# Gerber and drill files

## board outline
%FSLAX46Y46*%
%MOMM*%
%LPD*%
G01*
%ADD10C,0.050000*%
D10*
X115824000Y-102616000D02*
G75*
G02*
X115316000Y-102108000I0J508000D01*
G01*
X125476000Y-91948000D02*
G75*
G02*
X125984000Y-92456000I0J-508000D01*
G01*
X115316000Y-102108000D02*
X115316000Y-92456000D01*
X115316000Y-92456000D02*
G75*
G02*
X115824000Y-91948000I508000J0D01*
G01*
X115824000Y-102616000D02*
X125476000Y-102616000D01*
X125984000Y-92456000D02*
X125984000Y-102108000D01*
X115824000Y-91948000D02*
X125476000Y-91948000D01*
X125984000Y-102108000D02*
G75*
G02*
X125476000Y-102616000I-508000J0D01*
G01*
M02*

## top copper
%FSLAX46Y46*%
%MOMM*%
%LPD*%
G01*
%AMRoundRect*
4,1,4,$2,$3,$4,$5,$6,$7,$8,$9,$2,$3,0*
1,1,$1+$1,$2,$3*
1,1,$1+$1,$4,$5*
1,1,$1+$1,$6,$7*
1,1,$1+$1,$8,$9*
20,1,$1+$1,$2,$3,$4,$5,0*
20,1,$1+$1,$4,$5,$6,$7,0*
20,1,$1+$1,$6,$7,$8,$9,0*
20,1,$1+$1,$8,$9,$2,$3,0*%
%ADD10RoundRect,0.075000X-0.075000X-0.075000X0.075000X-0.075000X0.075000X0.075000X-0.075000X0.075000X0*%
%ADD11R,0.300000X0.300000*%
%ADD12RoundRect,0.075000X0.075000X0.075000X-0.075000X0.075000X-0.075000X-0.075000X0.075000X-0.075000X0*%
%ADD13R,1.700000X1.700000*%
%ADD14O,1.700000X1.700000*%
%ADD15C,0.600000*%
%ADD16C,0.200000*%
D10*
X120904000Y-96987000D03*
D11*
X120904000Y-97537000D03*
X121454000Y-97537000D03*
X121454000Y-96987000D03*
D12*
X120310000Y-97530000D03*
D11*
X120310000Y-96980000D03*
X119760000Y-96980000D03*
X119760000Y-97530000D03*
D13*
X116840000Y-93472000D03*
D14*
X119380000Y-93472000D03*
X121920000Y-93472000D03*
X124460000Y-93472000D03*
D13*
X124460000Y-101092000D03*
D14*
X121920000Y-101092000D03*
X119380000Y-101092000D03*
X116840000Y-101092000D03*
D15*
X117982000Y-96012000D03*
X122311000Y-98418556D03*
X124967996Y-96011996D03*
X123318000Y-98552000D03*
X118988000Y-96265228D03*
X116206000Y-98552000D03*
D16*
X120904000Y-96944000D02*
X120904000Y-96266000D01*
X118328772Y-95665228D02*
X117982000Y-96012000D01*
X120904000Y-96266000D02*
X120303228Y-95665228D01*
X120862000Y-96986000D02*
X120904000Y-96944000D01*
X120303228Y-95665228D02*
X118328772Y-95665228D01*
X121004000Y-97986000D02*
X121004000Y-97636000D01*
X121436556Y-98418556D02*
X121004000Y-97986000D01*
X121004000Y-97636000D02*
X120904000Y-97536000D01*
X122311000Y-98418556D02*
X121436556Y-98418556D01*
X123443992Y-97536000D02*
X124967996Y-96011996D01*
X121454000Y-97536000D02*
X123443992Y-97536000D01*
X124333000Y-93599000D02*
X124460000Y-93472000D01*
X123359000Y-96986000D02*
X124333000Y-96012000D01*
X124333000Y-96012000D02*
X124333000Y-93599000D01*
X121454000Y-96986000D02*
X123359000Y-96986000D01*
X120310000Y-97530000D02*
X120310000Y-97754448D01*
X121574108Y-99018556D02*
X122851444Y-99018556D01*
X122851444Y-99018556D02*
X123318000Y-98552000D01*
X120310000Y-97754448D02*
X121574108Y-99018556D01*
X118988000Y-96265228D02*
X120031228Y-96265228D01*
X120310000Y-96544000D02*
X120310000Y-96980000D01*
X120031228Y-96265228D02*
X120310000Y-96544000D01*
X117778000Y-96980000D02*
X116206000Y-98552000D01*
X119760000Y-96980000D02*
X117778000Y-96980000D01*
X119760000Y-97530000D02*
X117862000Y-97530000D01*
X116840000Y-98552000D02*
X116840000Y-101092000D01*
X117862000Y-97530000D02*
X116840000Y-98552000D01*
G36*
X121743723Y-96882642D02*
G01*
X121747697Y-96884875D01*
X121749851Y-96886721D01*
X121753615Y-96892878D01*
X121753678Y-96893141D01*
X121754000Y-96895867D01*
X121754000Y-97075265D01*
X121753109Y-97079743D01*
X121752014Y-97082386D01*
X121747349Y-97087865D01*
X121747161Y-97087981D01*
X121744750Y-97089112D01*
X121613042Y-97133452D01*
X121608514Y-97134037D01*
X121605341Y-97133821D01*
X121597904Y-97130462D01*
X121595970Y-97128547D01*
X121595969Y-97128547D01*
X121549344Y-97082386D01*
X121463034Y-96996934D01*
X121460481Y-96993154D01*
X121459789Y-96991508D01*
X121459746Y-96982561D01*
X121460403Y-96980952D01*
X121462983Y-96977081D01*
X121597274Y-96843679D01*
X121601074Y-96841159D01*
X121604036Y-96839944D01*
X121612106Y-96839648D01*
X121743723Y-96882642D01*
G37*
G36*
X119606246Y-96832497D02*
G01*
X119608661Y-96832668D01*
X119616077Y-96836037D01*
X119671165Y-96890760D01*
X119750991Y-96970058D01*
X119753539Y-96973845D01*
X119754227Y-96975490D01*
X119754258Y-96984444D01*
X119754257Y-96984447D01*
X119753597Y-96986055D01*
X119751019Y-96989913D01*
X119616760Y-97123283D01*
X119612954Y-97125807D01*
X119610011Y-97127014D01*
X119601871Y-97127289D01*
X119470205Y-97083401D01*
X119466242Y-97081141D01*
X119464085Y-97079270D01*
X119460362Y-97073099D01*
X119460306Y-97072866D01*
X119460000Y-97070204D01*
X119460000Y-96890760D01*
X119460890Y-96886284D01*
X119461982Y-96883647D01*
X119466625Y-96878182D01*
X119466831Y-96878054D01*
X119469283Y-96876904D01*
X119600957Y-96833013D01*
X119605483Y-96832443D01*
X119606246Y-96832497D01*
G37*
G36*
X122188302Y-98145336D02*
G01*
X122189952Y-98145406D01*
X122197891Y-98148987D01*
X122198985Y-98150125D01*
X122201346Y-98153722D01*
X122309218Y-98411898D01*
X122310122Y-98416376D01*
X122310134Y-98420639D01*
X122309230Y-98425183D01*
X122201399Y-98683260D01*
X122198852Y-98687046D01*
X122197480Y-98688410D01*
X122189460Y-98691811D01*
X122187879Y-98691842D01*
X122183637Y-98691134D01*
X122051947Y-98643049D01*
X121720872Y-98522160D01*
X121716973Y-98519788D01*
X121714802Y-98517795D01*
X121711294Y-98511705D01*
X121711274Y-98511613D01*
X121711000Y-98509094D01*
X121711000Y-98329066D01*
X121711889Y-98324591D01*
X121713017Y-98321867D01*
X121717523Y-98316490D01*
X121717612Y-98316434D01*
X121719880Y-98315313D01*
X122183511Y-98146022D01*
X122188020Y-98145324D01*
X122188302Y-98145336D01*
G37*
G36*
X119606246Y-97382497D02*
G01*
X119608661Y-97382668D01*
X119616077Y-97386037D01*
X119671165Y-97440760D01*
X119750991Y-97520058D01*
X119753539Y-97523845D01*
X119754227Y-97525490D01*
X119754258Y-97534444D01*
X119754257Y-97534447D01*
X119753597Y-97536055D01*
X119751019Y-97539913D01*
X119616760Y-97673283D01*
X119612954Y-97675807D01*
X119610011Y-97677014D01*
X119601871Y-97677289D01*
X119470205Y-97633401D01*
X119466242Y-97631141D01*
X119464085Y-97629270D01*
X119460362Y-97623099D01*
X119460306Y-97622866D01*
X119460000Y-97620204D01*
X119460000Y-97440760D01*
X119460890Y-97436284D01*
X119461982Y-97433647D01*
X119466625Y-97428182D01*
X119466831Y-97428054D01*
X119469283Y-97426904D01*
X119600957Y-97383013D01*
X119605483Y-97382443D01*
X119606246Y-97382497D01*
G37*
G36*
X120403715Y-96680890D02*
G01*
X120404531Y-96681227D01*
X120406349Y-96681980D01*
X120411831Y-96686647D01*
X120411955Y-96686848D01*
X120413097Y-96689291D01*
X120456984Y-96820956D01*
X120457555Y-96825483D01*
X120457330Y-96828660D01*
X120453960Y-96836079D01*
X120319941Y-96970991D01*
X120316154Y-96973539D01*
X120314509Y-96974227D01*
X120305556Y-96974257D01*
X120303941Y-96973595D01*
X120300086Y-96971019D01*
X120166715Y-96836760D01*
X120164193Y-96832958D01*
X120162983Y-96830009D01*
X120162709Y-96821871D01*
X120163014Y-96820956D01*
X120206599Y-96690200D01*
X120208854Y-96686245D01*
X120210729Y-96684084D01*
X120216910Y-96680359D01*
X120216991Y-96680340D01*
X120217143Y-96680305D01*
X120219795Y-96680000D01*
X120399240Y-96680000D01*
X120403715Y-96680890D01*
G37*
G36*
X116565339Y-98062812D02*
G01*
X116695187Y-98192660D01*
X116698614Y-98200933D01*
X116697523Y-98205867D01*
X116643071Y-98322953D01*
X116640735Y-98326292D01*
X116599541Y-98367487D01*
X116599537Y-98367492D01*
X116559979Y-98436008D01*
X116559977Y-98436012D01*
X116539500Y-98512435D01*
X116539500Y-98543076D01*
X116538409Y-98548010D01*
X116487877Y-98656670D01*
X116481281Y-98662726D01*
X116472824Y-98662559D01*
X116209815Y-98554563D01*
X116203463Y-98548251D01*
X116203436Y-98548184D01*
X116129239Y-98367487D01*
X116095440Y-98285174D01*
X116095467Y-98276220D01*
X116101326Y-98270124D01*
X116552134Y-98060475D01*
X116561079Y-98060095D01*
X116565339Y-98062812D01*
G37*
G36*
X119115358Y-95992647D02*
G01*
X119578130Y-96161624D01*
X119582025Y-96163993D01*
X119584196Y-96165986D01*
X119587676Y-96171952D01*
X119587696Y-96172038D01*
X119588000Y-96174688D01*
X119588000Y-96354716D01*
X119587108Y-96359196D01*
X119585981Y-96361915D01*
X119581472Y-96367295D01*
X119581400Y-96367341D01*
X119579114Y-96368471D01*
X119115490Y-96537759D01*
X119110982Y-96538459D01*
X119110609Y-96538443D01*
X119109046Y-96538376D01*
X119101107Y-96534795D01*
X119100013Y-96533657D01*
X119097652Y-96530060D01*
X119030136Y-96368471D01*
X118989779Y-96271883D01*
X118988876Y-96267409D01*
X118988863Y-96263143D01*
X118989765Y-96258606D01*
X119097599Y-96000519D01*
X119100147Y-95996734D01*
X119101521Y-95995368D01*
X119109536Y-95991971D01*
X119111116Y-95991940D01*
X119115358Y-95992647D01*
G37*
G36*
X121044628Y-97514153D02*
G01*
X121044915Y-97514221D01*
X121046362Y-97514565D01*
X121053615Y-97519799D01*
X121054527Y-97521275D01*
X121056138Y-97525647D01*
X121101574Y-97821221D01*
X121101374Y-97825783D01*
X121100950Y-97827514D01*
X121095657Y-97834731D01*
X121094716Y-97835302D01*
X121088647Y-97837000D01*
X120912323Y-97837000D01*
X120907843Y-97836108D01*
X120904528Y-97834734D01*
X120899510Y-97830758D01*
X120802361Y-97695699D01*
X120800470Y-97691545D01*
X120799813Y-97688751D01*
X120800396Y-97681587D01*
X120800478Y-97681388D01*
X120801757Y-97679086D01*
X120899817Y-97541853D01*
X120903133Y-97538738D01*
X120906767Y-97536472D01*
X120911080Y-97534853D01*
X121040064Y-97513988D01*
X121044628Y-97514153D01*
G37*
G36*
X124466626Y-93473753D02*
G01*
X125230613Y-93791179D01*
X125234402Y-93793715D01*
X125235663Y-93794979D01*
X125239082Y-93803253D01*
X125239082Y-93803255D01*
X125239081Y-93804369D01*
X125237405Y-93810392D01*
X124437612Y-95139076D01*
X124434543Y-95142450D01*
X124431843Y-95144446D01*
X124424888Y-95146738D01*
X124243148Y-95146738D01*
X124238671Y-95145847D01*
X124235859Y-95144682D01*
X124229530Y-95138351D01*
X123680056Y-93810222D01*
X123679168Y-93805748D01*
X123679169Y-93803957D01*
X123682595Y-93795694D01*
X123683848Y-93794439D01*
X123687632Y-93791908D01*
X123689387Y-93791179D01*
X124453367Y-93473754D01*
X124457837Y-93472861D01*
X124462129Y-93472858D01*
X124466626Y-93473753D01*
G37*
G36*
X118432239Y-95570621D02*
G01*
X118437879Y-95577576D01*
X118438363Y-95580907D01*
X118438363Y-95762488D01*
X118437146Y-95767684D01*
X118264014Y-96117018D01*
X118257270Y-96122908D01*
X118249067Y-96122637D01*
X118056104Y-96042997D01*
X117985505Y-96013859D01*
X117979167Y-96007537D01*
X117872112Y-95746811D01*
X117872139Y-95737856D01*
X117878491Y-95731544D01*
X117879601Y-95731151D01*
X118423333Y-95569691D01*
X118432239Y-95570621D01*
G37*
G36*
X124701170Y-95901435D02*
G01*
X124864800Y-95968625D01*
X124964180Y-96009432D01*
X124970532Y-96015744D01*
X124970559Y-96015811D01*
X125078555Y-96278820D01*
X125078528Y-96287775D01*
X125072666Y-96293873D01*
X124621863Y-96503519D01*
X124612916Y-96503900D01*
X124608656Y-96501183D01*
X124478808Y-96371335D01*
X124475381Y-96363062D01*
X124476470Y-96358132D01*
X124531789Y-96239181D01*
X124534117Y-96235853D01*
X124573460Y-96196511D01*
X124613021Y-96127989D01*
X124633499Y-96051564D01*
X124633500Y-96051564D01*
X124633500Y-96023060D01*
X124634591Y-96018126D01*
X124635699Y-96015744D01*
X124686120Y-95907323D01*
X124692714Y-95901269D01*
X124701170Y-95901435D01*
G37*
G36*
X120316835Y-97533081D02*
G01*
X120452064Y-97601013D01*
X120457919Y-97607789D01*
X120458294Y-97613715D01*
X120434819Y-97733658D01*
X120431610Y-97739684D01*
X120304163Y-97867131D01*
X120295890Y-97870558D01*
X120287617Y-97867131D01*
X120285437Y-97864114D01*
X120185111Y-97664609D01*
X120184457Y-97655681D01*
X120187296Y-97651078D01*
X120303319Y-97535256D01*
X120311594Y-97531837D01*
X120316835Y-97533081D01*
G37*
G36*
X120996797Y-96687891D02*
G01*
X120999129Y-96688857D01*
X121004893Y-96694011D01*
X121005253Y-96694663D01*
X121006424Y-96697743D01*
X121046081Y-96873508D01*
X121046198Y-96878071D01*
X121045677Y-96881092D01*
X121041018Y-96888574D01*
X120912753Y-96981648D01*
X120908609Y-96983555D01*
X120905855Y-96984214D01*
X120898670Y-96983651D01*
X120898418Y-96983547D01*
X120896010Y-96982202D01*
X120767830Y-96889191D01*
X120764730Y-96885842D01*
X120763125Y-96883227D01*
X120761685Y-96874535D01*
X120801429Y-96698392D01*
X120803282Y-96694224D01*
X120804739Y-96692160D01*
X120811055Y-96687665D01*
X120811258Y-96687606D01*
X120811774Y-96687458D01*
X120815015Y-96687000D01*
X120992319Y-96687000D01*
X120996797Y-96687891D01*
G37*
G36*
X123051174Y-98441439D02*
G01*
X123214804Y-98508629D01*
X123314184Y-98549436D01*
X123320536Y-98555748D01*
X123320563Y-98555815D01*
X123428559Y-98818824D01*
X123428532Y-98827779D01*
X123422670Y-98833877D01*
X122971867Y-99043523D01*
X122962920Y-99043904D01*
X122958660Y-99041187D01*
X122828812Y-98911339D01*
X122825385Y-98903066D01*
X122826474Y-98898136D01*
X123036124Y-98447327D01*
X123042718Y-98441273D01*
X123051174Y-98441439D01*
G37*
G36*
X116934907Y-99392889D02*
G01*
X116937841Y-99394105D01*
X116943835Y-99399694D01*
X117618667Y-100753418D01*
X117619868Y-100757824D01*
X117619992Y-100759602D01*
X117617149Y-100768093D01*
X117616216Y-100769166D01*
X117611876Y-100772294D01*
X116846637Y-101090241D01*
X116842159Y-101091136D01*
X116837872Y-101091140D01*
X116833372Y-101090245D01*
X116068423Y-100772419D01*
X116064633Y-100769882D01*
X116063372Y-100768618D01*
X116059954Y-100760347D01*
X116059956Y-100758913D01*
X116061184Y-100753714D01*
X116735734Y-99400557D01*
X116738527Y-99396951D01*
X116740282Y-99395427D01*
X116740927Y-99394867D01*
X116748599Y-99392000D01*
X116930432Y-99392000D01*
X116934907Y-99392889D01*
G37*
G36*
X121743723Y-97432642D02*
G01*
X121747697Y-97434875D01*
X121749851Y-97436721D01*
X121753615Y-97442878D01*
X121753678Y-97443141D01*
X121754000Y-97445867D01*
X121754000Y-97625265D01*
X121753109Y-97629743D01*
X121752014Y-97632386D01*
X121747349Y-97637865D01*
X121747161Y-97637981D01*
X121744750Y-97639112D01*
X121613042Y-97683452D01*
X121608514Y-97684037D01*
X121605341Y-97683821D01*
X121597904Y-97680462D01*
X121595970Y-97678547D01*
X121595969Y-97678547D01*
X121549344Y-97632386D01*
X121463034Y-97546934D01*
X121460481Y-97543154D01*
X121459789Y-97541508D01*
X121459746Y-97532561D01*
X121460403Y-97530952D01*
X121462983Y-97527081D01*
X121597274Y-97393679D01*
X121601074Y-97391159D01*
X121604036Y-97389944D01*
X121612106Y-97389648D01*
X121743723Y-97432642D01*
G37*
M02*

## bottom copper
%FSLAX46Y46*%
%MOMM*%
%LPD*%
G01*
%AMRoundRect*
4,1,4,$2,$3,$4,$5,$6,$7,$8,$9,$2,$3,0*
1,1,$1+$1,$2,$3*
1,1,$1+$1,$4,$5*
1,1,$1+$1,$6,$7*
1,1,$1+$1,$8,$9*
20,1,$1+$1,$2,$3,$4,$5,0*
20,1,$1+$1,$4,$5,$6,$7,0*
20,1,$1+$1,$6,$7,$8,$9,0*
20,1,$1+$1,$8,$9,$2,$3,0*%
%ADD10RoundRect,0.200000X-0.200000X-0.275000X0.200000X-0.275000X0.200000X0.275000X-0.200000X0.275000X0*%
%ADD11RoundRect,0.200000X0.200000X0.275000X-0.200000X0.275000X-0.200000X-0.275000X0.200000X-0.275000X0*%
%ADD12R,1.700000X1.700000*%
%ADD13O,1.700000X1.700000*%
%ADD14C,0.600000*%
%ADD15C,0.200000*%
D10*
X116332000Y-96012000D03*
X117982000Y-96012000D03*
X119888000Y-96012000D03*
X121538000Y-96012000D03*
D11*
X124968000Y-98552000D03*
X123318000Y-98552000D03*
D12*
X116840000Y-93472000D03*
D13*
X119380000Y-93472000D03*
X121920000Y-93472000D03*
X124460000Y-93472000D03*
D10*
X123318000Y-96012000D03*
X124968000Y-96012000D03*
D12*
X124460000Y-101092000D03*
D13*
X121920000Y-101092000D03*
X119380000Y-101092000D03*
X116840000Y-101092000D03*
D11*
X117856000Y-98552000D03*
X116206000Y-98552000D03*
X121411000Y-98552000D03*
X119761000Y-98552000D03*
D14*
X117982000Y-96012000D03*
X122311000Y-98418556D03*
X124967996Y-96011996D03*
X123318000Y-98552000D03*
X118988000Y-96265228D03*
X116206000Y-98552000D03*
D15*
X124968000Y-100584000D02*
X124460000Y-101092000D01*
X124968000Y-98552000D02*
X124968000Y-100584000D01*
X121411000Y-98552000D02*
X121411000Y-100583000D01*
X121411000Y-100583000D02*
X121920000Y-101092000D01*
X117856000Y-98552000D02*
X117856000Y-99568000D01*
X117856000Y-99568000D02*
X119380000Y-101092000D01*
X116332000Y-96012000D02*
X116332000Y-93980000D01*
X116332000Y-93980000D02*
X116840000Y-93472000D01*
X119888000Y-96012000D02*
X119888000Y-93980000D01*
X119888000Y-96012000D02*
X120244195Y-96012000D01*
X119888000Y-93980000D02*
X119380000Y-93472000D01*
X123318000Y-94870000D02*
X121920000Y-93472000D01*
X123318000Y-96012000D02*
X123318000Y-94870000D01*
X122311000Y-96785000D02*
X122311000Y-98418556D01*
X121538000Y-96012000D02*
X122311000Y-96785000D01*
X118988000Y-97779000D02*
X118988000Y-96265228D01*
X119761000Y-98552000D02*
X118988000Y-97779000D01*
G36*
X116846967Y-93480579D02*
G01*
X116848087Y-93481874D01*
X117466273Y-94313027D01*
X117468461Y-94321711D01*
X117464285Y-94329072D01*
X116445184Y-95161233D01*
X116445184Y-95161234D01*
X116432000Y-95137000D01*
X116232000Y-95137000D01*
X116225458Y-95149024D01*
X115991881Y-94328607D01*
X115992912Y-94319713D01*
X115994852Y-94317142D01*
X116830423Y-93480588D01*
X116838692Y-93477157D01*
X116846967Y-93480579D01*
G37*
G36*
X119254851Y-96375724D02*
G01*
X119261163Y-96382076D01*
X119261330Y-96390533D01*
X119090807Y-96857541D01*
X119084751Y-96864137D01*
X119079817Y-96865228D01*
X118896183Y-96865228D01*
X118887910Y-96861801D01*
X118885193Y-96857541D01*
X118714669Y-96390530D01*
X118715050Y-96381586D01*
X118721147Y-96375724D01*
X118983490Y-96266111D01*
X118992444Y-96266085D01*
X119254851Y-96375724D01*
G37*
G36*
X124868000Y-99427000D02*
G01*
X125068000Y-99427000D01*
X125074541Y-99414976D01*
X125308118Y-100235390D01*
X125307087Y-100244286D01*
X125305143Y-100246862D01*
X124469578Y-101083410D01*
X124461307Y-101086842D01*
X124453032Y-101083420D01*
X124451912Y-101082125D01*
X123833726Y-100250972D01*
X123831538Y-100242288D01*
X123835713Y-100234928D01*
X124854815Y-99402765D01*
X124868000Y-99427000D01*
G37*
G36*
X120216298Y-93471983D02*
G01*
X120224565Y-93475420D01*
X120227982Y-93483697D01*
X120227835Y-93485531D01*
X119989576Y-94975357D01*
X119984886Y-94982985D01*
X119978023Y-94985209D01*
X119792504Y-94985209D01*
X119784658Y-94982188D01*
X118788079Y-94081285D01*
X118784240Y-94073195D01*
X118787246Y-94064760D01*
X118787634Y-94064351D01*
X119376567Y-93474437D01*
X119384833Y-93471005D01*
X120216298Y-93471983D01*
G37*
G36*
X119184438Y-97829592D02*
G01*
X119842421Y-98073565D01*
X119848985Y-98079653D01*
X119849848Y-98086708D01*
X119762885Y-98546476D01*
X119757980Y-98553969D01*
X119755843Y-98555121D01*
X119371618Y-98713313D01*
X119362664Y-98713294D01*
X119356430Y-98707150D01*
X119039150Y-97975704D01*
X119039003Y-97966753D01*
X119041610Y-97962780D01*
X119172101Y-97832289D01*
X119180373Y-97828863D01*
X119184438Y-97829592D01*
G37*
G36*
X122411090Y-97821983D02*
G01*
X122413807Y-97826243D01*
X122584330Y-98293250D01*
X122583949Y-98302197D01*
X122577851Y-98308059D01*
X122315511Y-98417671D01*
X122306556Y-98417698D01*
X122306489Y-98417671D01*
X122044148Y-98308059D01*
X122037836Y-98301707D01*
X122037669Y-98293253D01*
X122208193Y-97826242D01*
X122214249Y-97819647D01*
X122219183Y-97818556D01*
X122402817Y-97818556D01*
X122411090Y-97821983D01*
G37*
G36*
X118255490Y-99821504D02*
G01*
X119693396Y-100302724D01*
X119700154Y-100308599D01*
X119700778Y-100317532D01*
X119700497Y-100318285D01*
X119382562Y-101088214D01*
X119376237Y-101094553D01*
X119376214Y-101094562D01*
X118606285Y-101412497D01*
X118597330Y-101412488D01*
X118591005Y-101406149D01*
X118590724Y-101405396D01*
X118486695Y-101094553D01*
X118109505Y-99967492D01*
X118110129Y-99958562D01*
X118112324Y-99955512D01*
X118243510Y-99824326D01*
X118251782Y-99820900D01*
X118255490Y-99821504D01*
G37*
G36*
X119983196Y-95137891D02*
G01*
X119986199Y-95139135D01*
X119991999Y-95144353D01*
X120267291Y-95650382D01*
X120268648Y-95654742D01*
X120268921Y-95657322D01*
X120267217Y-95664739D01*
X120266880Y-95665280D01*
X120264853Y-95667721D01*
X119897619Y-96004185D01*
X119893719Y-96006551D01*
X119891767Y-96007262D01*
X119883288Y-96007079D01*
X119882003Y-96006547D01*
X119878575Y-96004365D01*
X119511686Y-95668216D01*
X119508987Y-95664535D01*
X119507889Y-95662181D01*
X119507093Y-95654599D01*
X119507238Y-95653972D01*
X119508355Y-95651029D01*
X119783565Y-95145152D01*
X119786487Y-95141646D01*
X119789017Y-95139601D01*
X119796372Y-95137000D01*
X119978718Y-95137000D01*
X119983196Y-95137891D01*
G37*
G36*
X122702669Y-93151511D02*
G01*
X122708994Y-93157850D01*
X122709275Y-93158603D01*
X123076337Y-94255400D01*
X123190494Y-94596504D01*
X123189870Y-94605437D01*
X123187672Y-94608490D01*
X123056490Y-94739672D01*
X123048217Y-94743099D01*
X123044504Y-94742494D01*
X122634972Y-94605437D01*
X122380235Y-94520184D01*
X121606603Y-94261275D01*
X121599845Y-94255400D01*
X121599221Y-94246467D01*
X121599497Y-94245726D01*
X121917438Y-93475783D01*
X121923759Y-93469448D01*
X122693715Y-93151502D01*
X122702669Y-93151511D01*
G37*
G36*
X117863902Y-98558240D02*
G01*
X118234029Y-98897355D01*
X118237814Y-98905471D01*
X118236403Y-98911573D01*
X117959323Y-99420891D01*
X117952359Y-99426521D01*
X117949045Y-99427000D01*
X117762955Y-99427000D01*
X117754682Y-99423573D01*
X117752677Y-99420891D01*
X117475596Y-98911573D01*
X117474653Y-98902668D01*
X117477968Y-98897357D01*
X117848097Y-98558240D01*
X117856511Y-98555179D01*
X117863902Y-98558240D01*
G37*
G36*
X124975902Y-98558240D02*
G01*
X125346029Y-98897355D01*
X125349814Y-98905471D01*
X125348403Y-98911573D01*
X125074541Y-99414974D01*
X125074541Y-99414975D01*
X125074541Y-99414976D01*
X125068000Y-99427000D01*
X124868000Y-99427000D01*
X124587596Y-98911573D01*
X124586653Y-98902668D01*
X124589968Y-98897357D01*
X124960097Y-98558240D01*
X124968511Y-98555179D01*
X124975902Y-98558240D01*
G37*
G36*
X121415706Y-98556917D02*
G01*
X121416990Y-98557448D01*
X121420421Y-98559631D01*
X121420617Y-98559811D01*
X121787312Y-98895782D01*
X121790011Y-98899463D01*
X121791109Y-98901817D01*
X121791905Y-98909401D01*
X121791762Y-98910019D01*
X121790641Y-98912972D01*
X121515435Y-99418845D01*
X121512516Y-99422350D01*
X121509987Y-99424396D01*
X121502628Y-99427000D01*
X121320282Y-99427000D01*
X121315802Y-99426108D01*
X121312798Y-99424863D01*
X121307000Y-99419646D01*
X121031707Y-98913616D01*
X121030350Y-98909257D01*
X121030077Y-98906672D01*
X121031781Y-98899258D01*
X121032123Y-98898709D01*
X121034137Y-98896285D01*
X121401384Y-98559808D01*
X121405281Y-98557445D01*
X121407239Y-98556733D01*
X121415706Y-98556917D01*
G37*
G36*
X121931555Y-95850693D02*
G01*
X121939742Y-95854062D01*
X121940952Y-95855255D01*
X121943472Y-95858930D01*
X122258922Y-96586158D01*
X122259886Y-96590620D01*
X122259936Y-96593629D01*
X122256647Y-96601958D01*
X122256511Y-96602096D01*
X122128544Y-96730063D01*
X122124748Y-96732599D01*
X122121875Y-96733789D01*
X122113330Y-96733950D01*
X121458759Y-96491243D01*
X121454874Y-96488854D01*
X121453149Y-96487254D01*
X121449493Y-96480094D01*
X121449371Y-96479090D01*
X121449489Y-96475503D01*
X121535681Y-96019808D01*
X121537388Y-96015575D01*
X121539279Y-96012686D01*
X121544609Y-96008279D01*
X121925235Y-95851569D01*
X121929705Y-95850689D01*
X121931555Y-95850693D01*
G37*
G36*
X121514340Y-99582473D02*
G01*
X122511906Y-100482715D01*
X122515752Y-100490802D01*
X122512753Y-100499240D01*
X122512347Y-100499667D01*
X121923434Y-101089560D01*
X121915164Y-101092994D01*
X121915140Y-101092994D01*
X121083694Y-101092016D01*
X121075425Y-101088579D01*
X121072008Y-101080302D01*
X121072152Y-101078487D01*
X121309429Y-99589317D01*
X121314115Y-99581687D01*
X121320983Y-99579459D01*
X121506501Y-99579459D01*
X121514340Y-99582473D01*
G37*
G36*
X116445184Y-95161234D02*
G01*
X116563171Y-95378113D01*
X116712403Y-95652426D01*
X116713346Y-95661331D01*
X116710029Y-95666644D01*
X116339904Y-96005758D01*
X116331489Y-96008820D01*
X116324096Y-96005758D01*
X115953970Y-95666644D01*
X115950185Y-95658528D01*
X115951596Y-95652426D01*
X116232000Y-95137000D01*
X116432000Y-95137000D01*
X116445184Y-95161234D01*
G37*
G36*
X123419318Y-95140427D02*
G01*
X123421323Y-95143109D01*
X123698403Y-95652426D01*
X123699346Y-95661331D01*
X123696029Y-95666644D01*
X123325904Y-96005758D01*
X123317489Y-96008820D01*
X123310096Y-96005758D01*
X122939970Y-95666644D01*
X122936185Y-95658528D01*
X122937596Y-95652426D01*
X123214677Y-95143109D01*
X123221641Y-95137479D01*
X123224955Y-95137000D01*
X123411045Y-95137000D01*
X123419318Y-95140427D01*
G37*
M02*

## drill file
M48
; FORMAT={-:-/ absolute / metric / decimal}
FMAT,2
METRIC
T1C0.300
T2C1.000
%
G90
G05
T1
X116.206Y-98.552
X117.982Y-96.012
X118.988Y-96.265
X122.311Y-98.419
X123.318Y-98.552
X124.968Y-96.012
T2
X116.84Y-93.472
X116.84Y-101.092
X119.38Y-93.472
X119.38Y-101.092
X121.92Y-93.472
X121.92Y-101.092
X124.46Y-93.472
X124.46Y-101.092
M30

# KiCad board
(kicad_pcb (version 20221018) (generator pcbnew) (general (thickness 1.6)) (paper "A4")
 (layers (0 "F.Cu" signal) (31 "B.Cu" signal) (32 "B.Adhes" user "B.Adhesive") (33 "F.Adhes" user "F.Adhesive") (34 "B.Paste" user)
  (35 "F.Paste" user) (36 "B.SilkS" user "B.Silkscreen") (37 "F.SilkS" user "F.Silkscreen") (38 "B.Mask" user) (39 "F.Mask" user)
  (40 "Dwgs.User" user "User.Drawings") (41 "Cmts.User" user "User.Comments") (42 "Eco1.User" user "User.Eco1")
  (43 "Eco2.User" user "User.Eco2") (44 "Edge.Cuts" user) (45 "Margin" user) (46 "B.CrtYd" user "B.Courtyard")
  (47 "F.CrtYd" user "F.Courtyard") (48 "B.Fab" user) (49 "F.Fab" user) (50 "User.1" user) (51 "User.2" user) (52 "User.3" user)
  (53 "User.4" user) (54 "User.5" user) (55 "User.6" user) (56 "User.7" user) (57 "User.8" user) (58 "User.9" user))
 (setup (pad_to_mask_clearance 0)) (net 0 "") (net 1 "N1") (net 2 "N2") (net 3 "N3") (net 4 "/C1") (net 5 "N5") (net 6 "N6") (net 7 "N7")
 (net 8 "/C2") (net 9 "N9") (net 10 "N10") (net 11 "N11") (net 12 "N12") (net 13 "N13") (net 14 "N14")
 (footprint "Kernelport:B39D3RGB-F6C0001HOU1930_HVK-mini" (layer "F.Cu") (at 121.179 97.262)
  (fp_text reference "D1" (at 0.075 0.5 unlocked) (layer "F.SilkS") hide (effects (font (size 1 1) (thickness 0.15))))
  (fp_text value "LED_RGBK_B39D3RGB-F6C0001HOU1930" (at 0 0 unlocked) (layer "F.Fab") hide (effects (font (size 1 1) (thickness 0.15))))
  (pad "1" smd roundrect (at -0.275 -0.275) (size 0.3 0.3) (layers "F.Cu" "F.Paste" "F.Mask") (roundrect_rratio 0.25) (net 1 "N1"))
  (pad "2" smd rect (at -0.275 0.275) (size 0.3 0.3) (layers "F.Cu" "F.Paste" "F.Mask") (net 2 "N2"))
  (pad "3" smd rect (at 0.275 0.275) (size 0.3 0.3) (layers "F.Cu" "F.Paste" "F.Mask") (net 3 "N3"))
  (pad "4" smd rect (at 0.275 -0.275) (size 0.3 0.3) (layers "F.Cu" "F.Paste" "F.Mask") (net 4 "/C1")))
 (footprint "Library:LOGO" (layer "F.Cu") (at 123.952 97.282)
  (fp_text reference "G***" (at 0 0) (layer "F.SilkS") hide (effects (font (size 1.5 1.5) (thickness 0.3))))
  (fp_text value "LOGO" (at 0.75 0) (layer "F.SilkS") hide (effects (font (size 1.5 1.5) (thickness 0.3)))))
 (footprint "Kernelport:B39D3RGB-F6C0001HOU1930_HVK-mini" (layer "F.Cu") (at 120.035 97.255 180)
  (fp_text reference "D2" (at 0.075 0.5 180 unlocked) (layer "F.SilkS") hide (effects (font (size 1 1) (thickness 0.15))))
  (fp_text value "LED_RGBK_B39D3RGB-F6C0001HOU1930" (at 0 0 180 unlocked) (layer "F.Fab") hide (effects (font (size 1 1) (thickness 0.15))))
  (pad "1" smd roundrect (at -0.275 -0.275 180) (size 0.3 0.3) (layers "F.Cu" "F.Paste" "F.Mask") (roundrect_rratio 0.25) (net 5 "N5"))
  (pad "2" smd rect (at -0.275 0.275 180) (size 0.3 0.3) (layers "F.Cu" "F.Paste" "F.Mask") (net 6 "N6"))
  (pad "3" smd rect (at 0.275 0.275 180) (size 0.3 0.3) (layers "F.Cu" "F.Paste" "F.Mask") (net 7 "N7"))
  (pad "4" smd rect (at 0.275 -0.275 180) (size 0.3 0.3) (layers "F.Cu" "F.Paste" "F.Mask") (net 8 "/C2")))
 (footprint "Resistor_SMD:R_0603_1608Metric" (layer "B.Cu") (at 117.157 96.012)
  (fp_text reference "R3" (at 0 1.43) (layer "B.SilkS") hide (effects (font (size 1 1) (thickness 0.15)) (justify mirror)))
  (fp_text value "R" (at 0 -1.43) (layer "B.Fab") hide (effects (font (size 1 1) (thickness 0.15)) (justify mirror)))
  (pad "1" smd roundrect (at -0.825 0) (size 0.8 0.95) (layers "B.Cu" "B.Paste" "B.Mask") (roundrect_rratio 0.25) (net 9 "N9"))
  (pad "2" smd roundrect (at 0.825 0) (size 0.8 0.95) (layers "B.Cu" "B.Paste" "B.Mask") (roundrect_rratio 0.25) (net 1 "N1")))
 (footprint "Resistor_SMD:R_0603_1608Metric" (layer "B.Cu") (at 120.713 96.012)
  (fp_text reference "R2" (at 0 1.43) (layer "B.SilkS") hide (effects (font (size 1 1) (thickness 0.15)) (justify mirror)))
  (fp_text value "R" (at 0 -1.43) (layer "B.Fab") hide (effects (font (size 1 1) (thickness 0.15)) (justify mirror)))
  (pad "1" smd roundrect (at -0.825 0) (size 0.8 0.95) (layers "B.Cu" "B.Paste" "B.Mask") (roundrect_rratio 0.25) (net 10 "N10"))
  (pad "2" smd roundrect (at 0.825 0) (size 0.8 0.95) (layers "B.Cu" "B.Paste" "B.Mask") (roundrect_rratio 0.25) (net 2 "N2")))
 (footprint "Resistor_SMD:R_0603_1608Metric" (layer "B.Cu") (at 124.143 98.552 180)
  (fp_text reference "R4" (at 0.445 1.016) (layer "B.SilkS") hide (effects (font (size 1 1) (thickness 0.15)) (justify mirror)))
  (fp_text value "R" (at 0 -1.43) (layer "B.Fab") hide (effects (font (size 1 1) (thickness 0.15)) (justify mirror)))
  (pad "1" smd roundrect (at -0.825 0 180) (size 0.8 0.95) (layers "B.Cu" "B.Paste" "B.Mask") (roundrect_rratio 0.25) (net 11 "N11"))
  (pad "2" smd roundrect (at 0.825 0 180) (size 0.8 0.95) (layers "B.Cu" "B.Paste" "B.Mask") (roundrect_rratio 0.25) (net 5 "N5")))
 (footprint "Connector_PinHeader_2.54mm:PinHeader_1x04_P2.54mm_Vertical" (layer "B.Cu") (at 116.84 93.472 -90)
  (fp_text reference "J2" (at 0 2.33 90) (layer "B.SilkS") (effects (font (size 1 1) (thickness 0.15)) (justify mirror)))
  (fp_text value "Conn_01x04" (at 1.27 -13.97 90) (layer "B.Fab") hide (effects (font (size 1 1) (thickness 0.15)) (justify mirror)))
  (pad "1" thru_hole rect (at 0 0 270) (size 1.7 1.7) (drill 1) (layers "*.Cu" "*.Mask") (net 9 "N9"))
  (pad "2" thru_hole oval (at 0 -2.54 270) (size 1.7 1.7) (drill 1) (layers "*.Cu" "*.Mask") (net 10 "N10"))
  (pad "3" thru_hole oval (at 0 -5.08 270) (size 1.7 1.7) (drill 1) (layers "*.Cu" "*.Mask") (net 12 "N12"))
  (pad "4" thru_hole oval (at 0 -7.62 270) (size 1.7 1.7) (drill 1) (layers "*.Cu" "*.Mask") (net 4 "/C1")))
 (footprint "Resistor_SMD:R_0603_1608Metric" (layer "B.Cu") (at 124.143 96.012)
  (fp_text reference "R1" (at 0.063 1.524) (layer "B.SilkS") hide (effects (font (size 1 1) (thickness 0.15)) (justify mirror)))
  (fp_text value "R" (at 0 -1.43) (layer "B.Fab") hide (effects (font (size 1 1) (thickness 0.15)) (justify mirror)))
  (pad "1" smd roundrect (at -0.825 0) (size 0.8 0.95) (layers "B.Cu" "B.Paste" "B.Mask") (roundrect_rratio 0.25) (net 12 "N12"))
  (pad "2" smd roundrect (at 0.825 0) (size 0.8 0.95) (layers "B.Cu" "B.Paste" "B.Mask") (roundrect_rratio 0.25) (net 3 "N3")))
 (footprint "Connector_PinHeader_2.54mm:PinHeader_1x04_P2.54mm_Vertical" (layer "B.Cu") (at 124.46 101.092 90)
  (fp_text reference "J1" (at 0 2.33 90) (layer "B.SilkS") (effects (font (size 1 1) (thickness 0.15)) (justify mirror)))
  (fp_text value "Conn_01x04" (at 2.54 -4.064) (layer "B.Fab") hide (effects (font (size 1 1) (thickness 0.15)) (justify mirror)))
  (pad "1" thru_hole rect (at 0 0 90) (size 1.7 1.7) (drill 1) (layers "*.Cu" "*.Mask") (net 11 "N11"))
  (pad "2" thru_hole oval (at 0 -2.54 90) (size 1.7 1.7) (drill 1) (layers "*.Cu" "*.Mask") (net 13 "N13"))
  (pad "3" thru_hole oval (at 0 -5.08 90) (size 1.7 1.7) (drill 1) (layers "*.Cu" "*.Mask") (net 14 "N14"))
  (pad "4" thru_hole oval (at 0 -7.62 90) (size 1.7 1.7) (drill 1) (layers "*.Cu" "*.Mask") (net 8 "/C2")))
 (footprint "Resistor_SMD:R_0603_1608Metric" (layer "B.Cu") (at 117.031 98.552 180)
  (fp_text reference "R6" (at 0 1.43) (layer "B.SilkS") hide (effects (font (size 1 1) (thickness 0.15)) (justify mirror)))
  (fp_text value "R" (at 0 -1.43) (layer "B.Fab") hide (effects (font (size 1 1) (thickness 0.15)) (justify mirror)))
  (pad "1" smd roundrect (at -0.825 0 180) (size 0.8 0.95) (layers "B.Cu" "B.Paste" "B.Mask") (roundrect_rratio 0.25) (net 14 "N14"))
  (pad "2" smd roundrect (at 0.825 0 180) (size 0.8 0.95) (layers "B.Cu" "B.Paste" "B.Mask") (roundrect_rratio 0.25) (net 7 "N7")))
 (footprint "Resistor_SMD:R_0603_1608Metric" (layer "B.Cu") (at 120.586 98.552 180)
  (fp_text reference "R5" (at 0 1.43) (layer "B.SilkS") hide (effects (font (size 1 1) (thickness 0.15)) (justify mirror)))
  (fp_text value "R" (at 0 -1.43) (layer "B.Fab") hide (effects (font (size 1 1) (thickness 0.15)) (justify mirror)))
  (pad "1" smd roundrect (at -0.825 0 180) (size 0.8 0.95) (layers "B.Cu" "B.Paste" "B.Mask") (roundrect_rratio 0.25) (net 13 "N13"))
  (pad "2" smd roundrect (at 0.825 0 180) (size 0.8 0.95) (layers "B.Cu" "B.Paste" "B.Mask") (roundrect_rratio 0.25) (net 6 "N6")))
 (gr_arc (start 115.824 102.616) (mid 115.46479 102.46721) (end 115.316 102.108) (stroke (width 0.05) (type default)) (layer "Edge.Cuts"))
 (gr_arc (start 125.476 91.948) (mid 125.83521 92.09679) (end 125.984 92.456) (stroke (width 0.05) (type default)) (layer "Edge.Cuts"))
 (gr_line (start 115.316 102.108) (end 115.316 92.456) (stroke (width 0.05) (type default)) (layer "Edge.Cuts"))
 (gr_arc (start 115.316 92.456) (mid 115.46479 92.09679) (end 115.824 91.948) (stroke (width 0.05) (type default)) (layer "Edge.Cuts"))
 (gr_line (start 115.824 102.616) (end 125.476 102.616) (stroke (width 0.05) (type default)) (layer "Edge.Cuts"))
 (gr_line (start 125.984 92.456) (end 125.984 102.108) (stroke (width 0.05) (type default)) (layer "Edge.Cuts"))
 (gr_line (start 115.824 91.948) (end 125.476 91.948) (stroke (width 0.05) (type default)) (layer "Edge.Cuts"))
 (gr_arc (start 125.984 102.108) (mid 125.83521 102.46721) (end 125.476 102.616) (stroke (width 0.05) (type default)) (layer "Edge.Cuts"))
 (segment (start 124.968 100.584) (end 124.46 101.092) (width 0.2) (layer "B.Cu") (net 11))
 (segment (start 124.968 98.552) (end 124.968 100.584) (width 0.2) (layer "B.Cu") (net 11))
 (segment (start 121.411 98.552) (end 121.411 100.583) (width 0.2) (layer "B.Cu") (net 13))
 (segment (start 121.411 100.583) (end 121.92 101.092) (width 0.2) (layer "B.Cu") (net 13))
 (segment (start 117.856 98.552) (end 117.856 99.568) (width 0.2) (layer "B.Cu") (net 14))
 (segment (start 117.856 99.568) (end 119.38 101.092) (width 0.2) (layer "B.Cu") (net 14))
 (segment (start 116.332 96.012) (end 116.332 93.98) (width 0.2) (layer "B.Cu") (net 9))
 (segment (start 116.332 93.98) (end 116.84 93.472) (width 0.2) (layer "B.Cu") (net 9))
 (segment (start 119.888 96.012) (end 119.888 93.98) (width 0.2) (layer "B.Cu") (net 10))
 (segment (start 119.888 96.012) (end 120.244195 96.012) (width 0.2) (layer "B.Cu") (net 10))
 (segment (start 119.888 93.98) (end 119.38 93.472) (width 0.2) (layer "B.Cu") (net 10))
 (segment (start 123.318 94.87) (end 121.92 93.472) (width 0.2) (layer "B.Cu") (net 12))
 (segment (start 123.318 96.012) (end 123.318 94.87) (width 0.2) (layer "B.Cu") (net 12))
 (segment (start 120.904 96.944) (end 120.904 96.266) (width 0.2) (layer "F.Cu") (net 1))
 (segment (start 118.328772 95.665228) (end 117.982 96.012) (width 0.2) (layer "F.Cu") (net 1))
 (segment (start 120.904 96.266) (end 120.303228 95.665228) (width 0.2) (layer "F.Cu") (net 1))
 (segment (start 120.862 96.986) (end 120.904 96.944) (width 0.2) (layer "F.Cu") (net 1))
 (segment (start 120.303228 95.665228) (end 118.328772 95.665228) (width 0.2) (layer "F.Cu") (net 1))
 (via (at 117.982 96.012) (size 0.6) (drill 0.3) (layers "F.Cu" "B.Cu") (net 1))
 (segment (start 121.004 97.986) (end 121.004 97.636) (width 0.2) (layer "F.Cu") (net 2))
 (segment (start 121.436556 98.418556) (end 121.004 97.986) (width 0.2) (layer "F.Cu") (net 2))
 (segment (start 121.004 97.636) (end 120.904 97.536) (width 0.2) (layer "F.Cu") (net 2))
 (segment (start 122.311 98.418556) (end 121.436556 98.418556) (width 0.2) (layer "F.Cu") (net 2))
 (via (at 122.311 98.418556) (size 0.6) (drill 0.3) (layers "F.Cu" "B.Cu") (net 2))
 (segment (start 122.311 96.785) (end 122.311 98.418556) (width 0.2) (layer "B.Cu") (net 2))
 (segment (start 121.538 96.012) (end 122.311 96.785) (width 0.2) (layer "B.Cu") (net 2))
 (segment (start 123.443992 97.536) (end 124.967996 96.011996) (width 0.2) (layer "F.Cu") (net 3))
 (segment (start 121.454 97.536) (end 123.443992 97.536) (width 0.2) (layer "F.Cu") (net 3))
 (via (at 124.967996 96.011996) (size 0.6) (drill 0.3) (layers "F.Cu" "B.Cu") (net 3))
 (segment (start 124.333 93.599) (end 124.46 93.472) (width 0.2) (layer "F.Cu") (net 4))
 (segment (start 123.359 96.986) (end 124.333 96.012) (width 0.2) (layer "F.Cu") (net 4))
 (segment (start 124.333 96.012) (end 124.333 93.599) (width 0.2) (layer "F.Cu") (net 4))
 (segment (start 121.454 96.986) (end 123.359 96.986) (width 0.2) (layer "F.Cu") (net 4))
 (segment (start 120.31 97.53) (end 120.31 97.754448) (width 0.2) (layer "F.Cu") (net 5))
 (segment (start 121.574108 99.018556) (end 122.851444 99.018556) (width 0.2) (layer "F.Cu") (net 5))
 (segment (start 122.851444 99.018556) (end 123.318 98.552) (width 0.2) (layer "F.Cu") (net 5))
 (segment (start 120.31 97.754448) (end 121.574108 99.018556) (width 0.2) (layer "F.Cu") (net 5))
 (via (at 123.318 98.552) (size 0.6) (drill 0.3) (layers "F.Cu" "B.Cu") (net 5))
 (segment (start 118.988 96.265228) (end 120.031228 96.265228) (width 0.2) (layer "F.Cu") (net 6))
 (segment (start 120.31 96.544) (end 120.31 96.98) (width 0.2) (layer "F.Cu") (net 6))
 (segment (start 120.031228 96.265228) (end 120.31 96.544) (width 0.2) (layer "F.Cu") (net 6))
 (via (at 118.988 96.265228) (size 0.6) (drill 0.3) (layers "F.Cu" "B.Cu") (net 6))
 (segment (start 118.988 97.779) (end 118.988 96.265228) (width 0.2) (layer "B.Cu") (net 6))
 (segment (start 119.761 98.552) (end 118.988 97.779) (width 0.2) (layer "B.Cu") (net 6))
 (segment (start 117.778 96.98) (end 116.206 98.552) (width 0.2) (layer "F.Cu") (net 7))
 (segment (start 119.76 96.98) (end 117.778 96.98) (width 0.2) (layer "F.Cu") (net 7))
 (via (at 116.206 98.552) (size 0.6) (drill 0.3) (layers "F.Cu" "B.Cu") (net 7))
 (segment (start 119.76 97.53) (end 117.862 97.53) (width 0.2) (layer "F.Cu") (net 8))
 (segment (start 116.84 98.552) (end 116.84 101.092) (width 0.2) (layer "F.Cu") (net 8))
 (segment (start 117.862 97.53) (end 116.84 98.552) (width 0.2) (layer "F.Cu") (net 8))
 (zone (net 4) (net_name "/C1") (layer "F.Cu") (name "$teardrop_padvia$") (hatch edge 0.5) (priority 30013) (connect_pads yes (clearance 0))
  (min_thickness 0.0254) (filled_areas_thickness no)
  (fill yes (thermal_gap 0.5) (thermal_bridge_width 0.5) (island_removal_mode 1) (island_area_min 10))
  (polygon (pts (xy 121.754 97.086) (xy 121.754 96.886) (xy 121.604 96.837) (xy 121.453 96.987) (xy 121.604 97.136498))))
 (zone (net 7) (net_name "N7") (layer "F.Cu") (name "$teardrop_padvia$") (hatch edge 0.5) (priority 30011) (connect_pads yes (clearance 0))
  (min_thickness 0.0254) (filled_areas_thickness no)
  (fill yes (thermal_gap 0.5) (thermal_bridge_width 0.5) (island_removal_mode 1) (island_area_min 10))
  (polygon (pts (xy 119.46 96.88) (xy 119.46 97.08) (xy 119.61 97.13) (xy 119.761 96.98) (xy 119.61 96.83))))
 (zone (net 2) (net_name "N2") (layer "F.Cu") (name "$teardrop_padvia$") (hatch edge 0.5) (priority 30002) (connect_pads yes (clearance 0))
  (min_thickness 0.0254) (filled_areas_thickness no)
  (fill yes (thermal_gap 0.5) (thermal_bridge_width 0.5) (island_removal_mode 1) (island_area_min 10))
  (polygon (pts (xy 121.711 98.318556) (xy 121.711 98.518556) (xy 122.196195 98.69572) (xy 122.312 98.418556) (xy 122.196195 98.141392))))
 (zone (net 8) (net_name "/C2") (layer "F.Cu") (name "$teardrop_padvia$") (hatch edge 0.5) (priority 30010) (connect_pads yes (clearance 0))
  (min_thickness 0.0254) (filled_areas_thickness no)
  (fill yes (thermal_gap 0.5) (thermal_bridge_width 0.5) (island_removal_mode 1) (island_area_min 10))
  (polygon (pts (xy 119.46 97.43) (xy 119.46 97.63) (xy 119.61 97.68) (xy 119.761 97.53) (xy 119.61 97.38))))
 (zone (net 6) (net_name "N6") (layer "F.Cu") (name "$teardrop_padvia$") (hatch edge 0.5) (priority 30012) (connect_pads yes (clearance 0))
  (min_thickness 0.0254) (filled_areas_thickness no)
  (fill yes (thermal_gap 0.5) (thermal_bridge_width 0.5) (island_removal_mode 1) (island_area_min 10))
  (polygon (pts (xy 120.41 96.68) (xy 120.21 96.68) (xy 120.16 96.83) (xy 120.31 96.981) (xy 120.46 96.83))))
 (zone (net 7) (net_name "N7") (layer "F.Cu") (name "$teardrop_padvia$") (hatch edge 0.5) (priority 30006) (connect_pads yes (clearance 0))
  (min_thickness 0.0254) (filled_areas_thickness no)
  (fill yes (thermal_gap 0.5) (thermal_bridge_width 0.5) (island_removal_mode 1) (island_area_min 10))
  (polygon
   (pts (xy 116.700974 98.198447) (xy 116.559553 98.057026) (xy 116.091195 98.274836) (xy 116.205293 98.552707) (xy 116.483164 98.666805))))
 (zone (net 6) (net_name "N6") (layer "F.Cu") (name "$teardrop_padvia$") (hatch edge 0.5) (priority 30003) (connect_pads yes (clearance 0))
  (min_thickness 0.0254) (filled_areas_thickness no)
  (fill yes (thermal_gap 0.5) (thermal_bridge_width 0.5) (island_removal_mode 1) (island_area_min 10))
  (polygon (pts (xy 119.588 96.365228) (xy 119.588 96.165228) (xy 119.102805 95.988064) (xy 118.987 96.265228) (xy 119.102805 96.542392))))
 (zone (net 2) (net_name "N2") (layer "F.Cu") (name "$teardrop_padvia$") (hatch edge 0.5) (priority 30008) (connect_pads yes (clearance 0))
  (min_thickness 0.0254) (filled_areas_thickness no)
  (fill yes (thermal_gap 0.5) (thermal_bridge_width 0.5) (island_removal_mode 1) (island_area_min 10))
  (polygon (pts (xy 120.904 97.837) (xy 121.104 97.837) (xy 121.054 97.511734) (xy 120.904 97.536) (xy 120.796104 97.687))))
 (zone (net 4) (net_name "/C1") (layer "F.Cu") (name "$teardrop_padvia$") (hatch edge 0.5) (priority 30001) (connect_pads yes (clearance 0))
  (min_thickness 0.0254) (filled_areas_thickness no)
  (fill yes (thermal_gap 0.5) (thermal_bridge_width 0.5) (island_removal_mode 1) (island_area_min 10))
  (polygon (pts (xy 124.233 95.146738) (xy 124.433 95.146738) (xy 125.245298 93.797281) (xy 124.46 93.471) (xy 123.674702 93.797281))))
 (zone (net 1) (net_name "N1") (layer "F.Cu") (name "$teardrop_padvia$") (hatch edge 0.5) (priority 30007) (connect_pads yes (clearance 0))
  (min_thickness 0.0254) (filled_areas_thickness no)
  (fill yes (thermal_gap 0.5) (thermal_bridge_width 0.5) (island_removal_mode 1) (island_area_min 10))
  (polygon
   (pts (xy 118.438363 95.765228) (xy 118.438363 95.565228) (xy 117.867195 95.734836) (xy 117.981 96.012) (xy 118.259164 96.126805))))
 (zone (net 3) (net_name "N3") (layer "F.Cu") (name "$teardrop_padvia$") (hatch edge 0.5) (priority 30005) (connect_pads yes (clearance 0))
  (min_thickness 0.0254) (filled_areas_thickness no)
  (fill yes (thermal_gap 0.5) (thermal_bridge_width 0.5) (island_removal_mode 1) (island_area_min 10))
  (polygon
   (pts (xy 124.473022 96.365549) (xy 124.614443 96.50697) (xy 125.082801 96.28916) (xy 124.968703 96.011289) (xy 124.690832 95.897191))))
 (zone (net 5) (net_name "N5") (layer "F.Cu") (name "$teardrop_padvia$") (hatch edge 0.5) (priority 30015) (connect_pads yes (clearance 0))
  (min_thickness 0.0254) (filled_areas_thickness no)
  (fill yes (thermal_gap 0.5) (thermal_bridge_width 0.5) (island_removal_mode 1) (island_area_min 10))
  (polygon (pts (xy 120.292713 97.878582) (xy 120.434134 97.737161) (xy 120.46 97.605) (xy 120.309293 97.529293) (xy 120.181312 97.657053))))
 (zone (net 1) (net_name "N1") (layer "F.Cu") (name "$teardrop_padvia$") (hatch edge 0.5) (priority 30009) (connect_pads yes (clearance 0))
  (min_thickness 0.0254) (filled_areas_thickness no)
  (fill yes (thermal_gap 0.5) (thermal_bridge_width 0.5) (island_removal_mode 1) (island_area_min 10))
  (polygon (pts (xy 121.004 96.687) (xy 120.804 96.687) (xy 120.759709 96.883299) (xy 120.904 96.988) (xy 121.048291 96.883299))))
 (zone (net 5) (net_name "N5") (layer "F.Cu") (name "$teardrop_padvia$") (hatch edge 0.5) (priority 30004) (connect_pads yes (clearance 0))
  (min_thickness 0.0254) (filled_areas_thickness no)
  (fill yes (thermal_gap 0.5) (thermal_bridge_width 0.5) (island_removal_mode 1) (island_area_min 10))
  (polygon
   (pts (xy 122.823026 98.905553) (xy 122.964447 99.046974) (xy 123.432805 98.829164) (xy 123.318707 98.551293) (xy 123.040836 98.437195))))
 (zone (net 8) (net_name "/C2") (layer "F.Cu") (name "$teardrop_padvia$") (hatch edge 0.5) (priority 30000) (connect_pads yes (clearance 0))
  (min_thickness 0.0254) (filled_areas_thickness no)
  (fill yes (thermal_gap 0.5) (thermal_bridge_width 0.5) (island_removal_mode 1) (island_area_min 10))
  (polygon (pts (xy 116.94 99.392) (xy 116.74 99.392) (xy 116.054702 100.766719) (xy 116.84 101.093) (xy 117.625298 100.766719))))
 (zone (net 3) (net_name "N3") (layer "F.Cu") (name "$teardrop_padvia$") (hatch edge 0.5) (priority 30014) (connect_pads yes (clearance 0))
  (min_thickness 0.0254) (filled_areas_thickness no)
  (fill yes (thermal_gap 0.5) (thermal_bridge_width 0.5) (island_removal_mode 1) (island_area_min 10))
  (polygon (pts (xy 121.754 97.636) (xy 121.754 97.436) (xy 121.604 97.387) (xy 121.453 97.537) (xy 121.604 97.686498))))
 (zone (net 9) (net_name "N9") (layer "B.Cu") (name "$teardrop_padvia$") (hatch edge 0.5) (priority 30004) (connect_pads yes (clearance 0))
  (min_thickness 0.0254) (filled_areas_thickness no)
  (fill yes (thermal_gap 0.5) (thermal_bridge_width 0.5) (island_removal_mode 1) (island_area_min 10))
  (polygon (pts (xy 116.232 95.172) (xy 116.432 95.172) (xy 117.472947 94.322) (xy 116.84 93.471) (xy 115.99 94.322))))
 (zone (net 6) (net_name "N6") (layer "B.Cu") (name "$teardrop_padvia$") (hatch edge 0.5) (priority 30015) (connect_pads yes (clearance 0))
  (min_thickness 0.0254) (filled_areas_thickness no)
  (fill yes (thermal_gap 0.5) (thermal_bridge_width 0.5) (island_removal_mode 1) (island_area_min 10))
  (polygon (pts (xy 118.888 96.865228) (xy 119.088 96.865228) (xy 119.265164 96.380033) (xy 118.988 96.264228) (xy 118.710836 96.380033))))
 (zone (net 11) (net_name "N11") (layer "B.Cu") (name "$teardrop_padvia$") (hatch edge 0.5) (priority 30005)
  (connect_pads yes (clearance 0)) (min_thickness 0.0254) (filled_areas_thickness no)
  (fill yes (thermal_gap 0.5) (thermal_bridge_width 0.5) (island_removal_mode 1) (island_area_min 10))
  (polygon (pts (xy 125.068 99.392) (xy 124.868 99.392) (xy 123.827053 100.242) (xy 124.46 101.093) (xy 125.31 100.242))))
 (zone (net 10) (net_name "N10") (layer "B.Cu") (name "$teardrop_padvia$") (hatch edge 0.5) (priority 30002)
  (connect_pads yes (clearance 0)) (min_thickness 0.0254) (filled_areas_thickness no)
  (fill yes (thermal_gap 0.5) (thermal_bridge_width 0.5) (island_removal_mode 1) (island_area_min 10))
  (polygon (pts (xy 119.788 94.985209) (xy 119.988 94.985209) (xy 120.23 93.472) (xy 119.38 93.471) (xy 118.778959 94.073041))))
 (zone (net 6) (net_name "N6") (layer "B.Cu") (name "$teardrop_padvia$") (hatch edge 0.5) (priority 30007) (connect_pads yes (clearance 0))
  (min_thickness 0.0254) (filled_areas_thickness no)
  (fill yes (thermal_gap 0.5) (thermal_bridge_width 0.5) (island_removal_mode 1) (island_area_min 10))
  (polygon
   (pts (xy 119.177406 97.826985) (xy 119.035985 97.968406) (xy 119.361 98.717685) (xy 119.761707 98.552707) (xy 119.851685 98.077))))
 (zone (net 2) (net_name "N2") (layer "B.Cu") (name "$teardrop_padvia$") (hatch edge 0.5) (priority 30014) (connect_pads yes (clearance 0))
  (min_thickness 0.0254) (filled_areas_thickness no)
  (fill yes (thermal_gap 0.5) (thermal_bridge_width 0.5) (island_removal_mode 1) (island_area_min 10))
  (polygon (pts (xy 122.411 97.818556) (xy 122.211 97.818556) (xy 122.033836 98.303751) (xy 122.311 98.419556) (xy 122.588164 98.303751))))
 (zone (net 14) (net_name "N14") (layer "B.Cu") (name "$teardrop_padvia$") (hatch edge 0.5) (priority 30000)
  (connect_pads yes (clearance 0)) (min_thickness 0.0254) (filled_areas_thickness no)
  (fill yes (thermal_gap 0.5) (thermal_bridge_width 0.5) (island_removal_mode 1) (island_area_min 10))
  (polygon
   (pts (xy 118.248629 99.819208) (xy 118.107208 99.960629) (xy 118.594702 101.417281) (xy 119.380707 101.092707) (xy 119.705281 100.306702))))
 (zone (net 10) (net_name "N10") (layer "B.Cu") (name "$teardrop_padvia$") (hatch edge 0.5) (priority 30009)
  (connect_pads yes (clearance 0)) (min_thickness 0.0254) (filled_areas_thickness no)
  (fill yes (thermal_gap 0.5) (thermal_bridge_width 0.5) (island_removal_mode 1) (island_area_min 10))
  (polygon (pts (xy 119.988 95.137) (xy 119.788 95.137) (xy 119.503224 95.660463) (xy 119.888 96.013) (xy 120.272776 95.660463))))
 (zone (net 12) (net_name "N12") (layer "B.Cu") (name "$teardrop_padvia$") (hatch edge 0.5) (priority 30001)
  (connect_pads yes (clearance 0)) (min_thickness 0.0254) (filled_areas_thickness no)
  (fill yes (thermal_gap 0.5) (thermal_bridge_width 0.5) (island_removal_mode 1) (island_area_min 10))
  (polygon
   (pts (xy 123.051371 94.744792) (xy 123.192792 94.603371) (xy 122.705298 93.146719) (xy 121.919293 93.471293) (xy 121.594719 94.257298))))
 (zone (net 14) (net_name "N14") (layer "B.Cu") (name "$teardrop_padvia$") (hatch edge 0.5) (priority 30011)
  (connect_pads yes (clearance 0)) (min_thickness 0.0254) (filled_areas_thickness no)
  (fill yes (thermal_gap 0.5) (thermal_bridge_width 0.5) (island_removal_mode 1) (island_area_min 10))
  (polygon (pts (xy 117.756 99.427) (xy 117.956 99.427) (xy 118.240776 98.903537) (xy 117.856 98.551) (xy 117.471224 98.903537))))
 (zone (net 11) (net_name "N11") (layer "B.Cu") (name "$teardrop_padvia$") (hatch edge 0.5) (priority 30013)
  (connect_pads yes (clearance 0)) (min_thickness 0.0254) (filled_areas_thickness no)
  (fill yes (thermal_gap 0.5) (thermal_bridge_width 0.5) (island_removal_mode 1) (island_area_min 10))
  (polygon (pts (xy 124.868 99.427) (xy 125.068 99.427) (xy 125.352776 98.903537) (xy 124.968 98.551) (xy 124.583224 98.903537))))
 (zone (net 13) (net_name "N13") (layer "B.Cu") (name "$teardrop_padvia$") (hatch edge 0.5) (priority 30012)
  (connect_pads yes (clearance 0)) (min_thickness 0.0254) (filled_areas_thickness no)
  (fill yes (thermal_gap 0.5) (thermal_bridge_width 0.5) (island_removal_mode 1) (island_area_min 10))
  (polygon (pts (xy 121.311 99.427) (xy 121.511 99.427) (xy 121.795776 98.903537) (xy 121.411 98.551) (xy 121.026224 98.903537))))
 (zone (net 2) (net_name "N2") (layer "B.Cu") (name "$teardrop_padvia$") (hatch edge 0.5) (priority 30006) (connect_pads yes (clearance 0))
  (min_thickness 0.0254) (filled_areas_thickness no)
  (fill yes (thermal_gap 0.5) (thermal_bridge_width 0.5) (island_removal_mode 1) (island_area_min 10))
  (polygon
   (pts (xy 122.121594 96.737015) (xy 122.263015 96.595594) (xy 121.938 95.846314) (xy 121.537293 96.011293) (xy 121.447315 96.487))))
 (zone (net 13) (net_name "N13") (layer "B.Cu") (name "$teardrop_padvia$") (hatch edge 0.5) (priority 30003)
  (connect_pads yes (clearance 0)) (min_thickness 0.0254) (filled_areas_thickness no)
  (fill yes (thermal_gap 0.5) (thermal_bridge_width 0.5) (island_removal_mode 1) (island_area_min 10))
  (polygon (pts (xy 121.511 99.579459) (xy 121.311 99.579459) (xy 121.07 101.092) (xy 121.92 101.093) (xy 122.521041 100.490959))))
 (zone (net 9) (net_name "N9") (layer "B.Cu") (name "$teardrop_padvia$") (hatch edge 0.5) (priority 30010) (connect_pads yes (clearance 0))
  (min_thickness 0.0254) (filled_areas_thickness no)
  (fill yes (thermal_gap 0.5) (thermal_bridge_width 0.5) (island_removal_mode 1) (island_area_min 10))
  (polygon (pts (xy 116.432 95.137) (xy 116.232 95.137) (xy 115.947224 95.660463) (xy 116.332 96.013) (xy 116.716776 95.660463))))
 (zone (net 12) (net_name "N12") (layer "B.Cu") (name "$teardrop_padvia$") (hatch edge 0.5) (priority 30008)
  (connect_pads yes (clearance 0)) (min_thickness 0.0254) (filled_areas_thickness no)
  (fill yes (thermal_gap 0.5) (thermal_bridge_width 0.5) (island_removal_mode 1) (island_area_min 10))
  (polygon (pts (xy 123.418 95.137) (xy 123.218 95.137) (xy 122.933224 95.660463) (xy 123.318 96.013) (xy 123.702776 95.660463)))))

